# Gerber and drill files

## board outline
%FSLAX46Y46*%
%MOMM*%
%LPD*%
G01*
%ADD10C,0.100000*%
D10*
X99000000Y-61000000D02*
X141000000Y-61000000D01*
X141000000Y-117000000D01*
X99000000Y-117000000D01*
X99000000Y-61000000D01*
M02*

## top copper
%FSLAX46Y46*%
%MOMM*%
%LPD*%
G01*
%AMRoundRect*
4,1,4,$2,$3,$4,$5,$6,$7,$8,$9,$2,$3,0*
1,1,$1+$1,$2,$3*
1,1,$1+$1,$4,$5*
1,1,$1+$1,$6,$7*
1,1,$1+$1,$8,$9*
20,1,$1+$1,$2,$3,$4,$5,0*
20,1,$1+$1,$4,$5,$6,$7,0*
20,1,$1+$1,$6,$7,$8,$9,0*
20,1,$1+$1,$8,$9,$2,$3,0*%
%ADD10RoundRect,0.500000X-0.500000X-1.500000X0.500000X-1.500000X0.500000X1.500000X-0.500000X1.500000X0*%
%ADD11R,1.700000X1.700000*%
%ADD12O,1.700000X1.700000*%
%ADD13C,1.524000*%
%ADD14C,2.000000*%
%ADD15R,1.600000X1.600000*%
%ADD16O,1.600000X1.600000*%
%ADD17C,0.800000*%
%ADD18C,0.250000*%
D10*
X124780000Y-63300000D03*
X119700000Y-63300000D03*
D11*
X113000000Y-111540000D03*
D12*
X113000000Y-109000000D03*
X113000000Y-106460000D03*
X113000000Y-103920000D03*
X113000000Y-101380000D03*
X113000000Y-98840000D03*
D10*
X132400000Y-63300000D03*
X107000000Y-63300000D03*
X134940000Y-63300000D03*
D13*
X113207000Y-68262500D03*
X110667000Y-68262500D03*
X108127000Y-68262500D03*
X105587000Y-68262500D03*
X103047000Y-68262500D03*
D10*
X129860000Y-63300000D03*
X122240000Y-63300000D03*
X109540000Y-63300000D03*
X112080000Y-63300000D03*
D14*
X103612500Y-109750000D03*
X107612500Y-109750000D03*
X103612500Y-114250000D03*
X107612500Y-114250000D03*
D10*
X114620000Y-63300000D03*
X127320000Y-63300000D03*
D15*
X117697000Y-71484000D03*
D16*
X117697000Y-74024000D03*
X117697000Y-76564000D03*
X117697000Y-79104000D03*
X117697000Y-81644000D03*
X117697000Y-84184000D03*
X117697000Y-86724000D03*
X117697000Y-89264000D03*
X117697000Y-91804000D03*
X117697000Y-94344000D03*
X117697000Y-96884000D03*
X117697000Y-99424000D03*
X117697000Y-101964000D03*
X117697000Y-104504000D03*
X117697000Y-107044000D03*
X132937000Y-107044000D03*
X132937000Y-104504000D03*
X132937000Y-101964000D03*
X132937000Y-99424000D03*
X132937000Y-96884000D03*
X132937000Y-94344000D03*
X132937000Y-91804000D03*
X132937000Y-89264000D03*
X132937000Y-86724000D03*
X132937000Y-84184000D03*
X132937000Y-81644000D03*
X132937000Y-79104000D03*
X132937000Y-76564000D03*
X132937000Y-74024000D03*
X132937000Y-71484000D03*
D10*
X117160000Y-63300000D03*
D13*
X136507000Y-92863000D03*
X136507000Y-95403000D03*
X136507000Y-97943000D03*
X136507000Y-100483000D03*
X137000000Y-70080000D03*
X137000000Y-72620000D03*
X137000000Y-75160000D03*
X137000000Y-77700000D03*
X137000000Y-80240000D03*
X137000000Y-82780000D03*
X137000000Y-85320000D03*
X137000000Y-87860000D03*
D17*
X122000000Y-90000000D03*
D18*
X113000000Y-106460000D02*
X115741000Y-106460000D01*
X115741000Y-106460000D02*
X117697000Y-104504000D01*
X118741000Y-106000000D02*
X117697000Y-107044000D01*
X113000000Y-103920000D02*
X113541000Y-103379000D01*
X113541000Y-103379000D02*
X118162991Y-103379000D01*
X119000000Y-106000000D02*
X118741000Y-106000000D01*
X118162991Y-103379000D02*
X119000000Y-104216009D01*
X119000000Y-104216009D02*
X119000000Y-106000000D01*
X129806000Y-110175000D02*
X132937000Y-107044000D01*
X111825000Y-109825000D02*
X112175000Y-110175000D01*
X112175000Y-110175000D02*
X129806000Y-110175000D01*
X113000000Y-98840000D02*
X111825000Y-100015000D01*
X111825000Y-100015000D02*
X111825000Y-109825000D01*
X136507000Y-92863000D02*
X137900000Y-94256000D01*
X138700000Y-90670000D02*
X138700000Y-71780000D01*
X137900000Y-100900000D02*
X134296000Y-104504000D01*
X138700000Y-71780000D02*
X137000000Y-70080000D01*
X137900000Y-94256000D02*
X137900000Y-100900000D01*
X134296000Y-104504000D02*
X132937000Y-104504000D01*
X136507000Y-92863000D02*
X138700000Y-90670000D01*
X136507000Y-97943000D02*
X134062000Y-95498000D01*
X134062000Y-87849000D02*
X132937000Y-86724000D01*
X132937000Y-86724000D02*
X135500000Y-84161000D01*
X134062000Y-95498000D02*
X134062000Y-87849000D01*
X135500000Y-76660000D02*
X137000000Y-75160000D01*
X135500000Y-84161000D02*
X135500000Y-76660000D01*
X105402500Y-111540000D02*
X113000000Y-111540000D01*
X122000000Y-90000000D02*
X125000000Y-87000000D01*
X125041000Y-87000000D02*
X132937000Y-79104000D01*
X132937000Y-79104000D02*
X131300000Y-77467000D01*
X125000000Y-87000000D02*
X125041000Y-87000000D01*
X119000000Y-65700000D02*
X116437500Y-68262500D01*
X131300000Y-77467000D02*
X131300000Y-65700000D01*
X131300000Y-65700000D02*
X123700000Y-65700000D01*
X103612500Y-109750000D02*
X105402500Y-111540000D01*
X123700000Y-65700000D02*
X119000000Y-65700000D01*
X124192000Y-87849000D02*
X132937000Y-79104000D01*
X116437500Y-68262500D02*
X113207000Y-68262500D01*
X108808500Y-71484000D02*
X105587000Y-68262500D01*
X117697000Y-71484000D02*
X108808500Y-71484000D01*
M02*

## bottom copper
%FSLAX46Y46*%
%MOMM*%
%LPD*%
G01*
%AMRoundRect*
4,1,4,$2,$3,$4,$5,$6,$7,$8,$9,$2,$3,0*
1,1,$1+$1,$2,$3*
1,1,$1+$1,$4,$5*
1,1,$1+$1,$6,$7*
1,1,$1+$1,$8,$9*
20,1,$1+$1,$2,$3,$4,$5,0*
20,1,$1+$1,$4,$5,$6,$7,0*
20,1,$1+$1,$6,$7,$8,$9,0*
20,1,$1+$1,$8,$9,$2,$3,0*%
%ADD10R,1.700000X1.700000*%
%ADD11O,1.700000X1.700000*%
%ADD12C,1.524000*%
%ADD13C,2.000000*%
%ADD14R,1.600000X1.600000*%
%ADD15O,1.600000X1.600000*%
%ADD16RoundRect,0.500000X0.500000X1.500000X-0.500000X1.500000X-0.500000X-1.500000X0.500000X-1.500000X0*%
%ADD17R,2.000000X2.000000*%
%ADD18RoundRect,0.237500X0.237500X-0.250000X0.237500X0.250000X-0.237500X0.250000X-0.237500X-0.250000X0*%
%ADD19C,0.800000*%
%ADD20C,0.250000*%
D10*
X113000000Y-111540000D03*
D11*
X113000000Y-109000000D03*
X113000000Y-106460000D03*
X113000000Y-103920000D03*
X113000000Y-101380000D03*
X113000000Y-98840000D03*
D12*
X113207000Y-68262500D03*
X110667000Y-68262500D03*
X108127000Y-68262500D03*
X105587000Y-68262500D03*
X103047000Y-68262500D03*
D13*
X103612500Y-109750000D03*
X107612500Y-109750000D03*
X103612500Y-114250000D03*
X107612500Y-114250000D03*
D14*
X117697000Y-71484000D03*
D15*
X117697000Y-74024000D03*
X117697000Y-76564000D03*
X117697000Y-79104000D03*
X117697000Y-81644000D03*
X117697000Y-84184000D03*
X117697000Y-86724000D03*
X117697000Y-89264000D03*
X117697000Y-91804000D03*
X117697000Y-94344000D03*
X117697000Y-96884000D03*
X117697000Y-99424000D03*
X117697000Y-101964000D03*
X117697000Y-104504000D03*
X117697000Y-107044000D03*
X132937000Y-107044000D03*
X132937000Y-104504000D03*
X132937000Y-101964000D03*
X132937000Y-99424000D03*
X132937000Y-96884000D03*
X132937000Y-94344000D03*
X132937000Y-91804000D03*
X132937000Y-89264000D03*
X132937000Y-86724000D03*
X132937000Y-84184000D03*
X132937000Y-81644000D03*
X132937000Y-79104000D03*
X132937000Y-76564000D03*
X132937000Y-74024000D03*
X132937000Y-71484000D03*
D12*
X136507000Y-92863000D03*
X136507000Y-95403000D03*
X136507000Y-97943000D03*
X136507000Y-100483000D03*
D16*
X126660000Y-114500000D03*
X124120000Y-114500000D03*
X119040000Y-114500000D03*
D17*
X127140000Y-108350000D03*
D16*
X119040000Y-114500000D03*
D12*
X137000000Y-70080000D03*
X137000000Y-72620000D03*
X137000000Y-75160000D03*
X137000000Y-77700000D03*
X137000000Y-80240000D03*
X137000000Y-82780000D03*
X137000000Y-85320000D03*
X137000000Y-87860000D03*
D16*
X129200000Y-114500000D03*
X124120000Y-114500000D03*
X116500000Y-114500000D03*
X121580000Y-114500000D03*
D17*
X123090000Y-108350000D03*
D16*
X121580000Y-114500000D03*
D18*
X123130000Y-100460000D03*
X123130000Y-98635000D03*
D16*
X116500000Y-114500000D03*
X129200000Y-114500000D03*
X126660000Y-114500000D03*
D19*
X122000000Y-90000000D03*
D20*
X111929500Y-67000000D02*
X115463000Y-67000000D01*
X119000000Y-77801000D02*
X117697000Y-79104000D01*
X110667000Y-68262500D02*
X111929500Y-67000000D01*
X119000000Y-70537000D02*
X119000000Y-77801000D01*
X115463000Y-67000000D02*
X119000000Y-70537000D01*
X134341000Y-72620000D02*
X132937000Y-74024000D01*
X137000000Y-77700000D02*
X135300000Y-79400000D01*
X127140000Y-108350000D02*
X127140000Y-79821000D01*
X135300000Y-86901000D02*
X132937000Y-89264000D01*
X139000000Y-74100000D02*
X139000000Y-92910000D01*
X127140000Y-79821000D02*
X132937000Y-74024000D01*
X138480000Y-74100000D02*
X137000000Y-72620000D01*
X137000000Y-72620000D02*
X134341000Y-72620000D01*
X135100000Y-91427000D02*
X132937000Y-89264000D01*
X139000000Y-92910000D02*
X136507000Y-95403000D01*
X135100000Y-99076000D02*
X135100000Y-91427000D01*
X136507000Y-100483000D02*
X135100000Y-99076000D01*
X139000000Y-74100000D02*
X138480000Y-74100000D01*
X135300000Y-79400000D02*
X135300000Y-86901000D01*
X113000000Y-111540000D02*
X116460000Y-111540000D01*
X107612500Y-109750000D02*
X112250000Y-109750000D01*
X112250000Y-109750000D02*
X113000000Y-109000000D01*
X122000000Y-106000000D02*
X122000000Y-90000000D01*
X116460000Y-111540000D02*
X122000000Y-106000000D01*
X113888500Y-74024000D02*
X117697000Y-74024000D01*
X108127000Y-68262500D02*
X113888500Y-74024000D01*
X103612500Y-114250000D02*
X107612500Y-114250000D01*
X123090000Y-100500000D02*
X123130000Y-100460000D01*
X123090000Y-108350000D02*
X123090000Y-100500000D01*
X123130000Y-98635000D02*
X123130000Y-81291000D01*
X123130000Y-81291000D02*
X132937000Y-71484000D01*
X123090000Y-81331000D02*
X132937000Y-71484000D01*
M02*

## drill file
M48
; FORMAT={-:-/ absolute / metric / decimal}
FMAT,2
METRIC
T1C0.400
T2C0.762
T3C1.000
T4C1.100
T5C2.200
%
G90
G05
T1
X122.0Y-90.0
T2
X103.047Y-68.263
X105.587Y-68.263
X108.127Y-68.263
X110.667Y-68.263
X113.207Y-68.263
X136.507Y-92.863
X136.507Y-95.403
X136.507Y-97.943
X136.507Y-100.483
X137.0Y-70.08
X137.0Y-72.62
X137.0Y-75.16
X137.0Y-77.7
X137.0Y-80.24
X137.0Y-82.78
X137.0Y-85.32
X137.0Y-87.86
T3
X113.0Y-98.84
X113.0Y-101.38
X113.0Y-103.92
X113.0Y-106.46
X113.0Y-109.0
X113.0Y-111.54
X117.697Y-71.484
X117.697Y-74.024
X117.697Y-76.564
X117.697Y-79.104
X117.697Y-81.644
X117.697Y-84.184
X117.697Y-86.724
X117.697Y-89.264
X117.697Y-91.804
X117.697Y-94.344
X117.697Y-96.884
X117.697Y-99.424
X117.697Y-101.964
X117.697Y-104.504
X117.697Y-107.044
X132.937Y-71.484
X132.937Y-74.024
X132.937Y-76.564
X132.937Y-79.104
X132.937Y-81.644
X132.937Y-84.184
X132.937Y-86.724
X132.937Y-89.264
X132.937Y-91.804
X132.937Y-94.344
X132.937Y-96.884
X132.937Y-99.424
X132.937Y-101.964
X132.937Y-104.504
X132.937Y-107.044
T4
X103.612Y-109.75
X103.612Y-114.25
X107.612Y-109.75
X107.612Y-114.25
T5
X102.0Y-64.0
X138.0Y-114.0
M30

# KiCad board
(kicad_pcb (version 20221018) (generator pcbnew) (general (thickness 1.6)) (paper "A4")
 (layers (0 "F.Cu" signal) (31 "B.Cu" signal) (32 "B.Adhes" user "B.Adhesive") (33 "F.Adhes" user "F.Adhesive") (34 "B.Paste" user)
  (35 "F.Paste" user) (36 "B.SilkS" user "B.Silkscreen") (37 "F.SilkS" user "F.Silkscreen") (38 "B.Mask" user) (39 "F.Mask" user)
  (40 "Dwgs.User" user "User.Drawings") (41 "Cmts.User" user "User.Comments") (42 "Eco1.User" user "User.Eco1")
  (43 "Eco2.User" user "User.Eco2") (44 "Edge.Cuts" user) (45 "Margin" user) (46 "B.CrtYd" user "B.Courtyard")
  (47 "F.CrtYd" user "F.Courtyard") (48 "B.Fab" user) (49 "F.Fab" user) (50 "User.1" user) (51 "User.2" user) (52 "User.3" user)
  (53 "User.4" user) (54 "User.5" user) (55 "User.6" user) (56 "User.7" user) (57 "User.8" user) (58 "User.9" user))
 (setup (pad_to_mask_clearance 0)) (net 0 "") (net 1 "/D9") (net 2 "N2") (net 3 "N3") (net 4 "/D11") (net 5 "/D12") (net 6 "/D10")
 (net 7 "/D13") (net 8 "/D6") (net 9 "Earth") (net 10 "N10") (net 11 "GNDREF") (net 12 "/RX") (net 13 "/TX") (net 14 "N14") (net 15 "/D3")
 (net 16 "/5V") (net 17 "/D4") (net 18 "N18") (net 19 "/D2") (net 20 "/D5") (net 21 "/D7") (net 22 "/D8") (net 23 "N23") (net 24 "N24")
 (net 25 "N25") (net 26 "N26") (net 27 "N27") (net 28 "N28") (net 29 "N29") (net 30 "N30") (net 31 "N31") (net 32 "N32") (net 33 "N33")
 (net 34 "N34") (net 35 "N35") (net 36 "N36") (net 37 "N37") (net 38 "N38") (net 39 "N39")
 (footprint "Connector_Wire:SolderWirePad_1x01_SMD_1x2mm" (layer "F.Cu") (at 124.78 63.3)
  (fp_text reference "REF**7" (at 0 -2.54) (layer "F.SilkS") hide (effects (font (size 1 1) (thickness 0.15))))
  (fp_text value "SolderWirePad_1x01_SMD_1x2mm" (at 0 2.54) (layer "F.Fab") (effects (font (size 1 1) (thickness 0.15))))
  (pad "1" smd roundrect (at 0 0) (size 2 4) (layers "F.Cu" "F.Paste" "F.Mask") (roundrect_rratio 0.25) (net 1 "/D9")))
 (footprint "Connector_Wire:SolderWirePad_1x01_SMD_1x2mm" (layer "F.Cu") (at 119.7 63.3)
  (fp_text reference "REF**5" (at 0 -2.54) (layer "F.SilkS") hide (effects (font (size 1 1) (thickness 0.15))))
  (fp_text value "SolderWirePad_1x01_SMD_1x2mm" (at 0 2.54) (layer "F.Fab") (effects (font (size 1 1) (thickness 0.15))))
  (pad "1" smd roundrect (at 0 0) (size 2 4) (layers "F.Cu" "F.Paste" "F.Mask") (roundrect_rratio 0.25)))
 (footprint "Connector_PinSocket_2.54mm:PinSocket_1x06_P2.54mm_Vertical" (layer "F.Cu") (at 113 111.54 180)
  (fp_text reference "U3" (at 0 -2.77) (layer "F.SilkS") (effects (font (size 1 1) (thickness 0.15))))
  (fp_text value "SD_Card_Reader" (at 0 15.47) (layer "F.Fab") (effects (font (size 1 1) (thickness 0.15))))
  (pad "1" thru_hole rect (at 0 0 180) (size 1.7 1.7) (drill 1) (layers "*.Cu" "*.Mask") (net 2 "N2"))
  (pad "2" thru_hole oval (at 0 2.54 180) (size 1.7 1.7) (drill 1) (layers "*.Cu" "*.Mask") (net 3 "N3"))
  (pad "3" thru_hole oval (at 0 5.08 180) (size 1.7 1.7) (drill 1) (layers "*.Cu" "*.Mask") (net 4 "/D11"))
  (pad "4" thru_hole oval (at 0 7.62 180) (size 1.7 1.7) (drill 1) (layers "*.Cu" "*.Mask") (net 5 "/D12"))
  (pad "5" thru_hole oval (at 0 10.16 180) (size 1.7 1.7) (drill 1) (layers "*.Cu" "*.Mask") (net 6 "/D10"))
  (pad "6" thru_hole oval (at 0 12.7 180) (size 1.7 1.7) (drill 1) (layers "*.Cu" "*.Mask") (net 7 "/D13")))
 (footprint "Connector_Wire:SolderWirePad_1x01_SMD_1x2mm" (layer "F.Cu") (at 132.4 63.3)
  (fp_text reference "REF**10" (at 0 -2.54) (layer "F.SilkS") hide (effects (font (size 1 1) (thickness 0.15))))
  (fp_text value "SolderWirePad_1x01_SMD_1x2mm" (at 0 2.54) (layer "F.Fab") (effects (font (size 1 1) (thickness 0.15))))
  (pad "1" smd roundrect (at 0 0) (size 2 4) (layers "F.Cu" "F.Paste" "F.Mask") (roundrect_rratio 0.25) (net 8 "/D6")))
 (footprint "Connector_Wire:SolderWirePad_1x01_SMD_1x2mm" (layer "F.Cu") (at 107 63.3)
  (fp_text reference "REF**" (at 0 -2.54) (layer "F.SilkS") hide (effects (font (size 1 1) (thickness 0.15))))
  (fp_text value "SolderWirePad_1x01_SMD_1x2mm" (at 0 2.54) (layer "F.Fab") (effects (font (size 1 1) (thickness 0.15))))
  (pad "1" smd roundrect (at 0 0) (size 2 4) (layers "F.Cu" "F.Paste" "F.Mask") (roundrect_rratio 0.25) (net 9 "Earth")))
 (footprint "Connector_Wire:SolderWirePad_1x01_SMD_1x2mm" (layer "F.Cu") (at 134.94 63.3)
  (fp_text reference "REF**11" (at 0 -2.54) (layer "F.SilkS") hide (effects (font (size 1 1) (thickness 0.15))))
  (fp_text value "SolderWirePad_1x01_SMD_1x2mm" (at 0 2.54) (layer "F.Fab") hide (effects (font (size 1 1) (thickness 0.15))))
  (pad "1" smd roundrect (at 0 0) (size 2 4) (layers "F.Cu" "F.Paste" "F.Mask") (roundrect_rratio 0.25)))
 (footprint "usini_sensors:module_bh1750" (layer "F.Cu") (at 103.047 68.2625 -90)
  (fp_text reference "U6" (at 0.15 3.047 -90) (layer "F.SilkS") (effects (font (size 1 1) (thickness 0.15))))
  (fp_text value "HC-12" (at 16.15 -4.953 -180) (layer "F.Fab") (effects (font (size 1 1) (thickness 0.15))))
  (pad "1" thru_hole circle (at 0 -10.16 270) (size 1.524 1.524) (drill 0.762) (layers "*.Cu" "*.Mask") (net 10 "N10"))
  (pad "2" thru_hole circle (at 0 -7.62 270) (size 1.524 1.524) (drill 0.762) (layers "*.Cu" "*.Mask") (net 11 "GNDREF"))
  (pad "3" thru_hole circle (at 0 -5.08 270) (size 1.524 1.524) (drill 0.762) (layers "*.Cu" "*.Mask") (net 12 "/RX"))
  (pad "4" thru_hole circle (at 0 -2.54 270) (size 1.524 1.524) (drill 0.762) (layers "*.Cu" "*.Mask") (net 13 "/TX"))
  (pad "5" thru_hole circle (at 0 0 270) (size 1.524 1.524) (drill 0.762) (layers "*.Cu" "*.Mask") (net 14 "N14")))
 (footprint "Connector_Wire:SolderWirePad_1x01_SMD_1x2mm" (layer "F.Cu") (at 129.86 63.3)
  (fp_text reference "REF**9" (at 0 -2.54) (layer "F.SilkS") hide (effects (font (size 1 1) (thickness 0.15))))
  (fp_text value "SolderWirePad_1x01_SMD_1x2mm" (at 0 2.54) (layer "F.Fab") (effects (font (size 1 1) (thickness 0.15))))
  (pad "1" smd roundrect (at 0 0) (size 2 4) (layers "F.Cu" "F.Paste" "F.Mask") (roundrect_rratio 0.25) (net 9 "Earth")))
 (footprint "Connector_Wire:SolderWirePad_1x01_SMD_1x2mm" (layer "F.Cu") (at 122.24 63.3)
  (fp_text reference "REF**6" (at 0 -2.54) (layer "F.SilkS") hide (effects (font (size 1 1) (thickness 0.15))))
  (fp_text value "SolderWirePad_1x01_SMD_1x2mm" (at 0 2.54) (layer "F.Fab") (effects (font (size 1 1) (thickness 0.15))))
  (pad "1" smd roundrect (at 0 0) (size 2 4) (layers "F.Cu" "F.Paste" "F.Mask") (roundrect_rratio 0.25) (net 9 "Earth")))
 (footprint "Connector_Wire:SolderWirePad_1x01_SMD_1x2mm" (layer "F.Cu") (at 109.54 63.3)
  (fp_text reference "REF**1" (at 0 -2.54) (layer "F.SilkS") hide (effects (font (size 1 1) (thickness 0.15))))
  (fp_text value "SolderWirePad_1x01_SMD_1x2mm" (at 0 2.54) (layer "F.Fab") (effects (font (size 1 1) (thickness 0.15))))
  (pad "1" smd roundrect (at 0 0) (size 2 4) (layers "F.Cu" "F.Paste" "F.Mask") (roundrect_rratio 0.25) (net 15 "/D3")))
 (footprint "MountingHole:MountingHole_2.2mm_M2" (layer "F.Cu") (at 138 114)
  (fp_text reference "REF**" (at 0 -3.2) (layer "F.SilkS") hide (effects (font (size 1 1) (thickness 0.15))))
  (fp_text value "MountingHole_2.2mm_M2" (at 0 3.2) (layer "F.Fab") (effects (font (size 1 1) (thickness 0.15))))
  (pad "" np_thru_hole circle (at 0 0) (size 2.2 2.2) (drill 2.2) (layers "*.Cu" "*.Mask")))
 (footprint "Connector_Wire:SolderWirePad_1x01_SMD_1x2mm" (layer "F.Cu") (at 112.08 63.3)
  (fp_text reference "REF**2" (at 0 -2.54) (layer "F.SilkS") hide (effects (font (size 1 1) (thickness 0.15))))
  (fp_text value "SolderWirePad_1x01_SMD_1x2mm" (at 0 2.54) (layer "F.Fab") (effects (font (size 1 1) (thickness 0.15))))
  (pad "1" smd roundrect (at 0 0) (size 2 4) (layers "F.Cu" "F.Paste" "F.Mask") (roundrect_rratio 0.25)))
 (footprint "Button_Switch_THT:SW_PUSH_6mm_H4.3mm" (layer "F.Cu") (at 101.1125 109.75)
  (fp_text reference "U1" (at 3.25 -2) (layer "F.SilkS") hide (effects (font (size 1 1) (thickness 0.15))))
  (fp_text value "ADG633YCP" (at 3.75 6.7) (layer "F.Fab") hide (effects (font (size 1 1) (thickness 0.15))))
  (pad "1" thru_hole circle (at 2.5 0 90) (size 2 2) (drill 1.1) (layers "*.Cu" "*.Mask") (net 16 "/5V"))
  (pad "1" thru_hole circle (at 6.5 0 90) (size 2 2) (drill 1.1) (layers "*.Cu" "*.Mask") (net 16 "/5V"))
  (pad "2" thru_hole circle (at 2.5 4.5 90) (size 2 2) (drill 1.1) (layers "*.Cu" "*.Mask") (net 8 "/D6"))
  (pad "2" thru_hole circle (at 6.5 4.5 90) (size 2 2) (drill 1.1) (layers "*.Cu" "*.Mask") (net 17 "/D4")))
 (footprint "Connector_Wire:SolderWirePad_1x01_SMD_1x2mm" (layer "F.Cu") (at 114.62 63.3)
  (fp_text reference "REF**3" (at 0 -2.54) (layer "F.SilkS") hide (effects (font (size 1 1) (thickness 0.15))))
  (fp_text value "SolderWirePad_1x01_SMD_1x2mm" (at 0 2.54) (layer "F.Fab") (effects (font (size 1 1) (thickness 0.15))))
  (pad "1" smd roundrect (at 0 0) (size 2 4) (layers "F.Cu" "F.Paste" "F.Mask") (roundrect_rratio 0.25) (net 9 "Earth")))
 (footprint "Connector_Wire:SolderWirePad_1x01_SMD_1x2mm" (layer "F.Cu") (at 127.32 63.3)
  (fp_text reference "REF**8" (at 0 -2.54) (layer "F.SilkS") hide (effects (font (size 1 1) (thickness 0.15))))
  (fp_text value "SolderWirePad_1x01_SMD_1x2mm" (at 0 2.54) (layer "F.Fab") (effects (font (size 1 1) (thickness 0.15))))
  (pad "1" smd roundrect (at 0 0) (size 2 4) (layers "F.Cu" "F.Paste" "F.Mask") (roundrect_rratio 0.25)))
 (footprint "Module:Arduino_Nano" (layer "F.Cu") (at 117.697 71.484)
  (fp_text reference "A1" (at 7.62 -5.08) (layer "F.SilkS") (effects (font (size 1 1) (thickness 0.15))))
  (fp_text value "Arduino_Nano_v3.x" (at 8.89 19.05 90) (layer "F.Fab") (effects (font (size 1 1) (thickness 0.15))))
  (pad "1" thru_hole rect (at 0 0) (size 1.6 1.6) (drill 1) (layers "*.Cu" "*.Mask") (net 13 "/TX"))
  (pad "2" thru_hole oval (at 0 2.54) (size 1.6 1.6) (drill 1) (layers "*.Cu" "*.Mask") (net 12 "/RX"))
  (pad "3" thru_hole oval (at 0 5.08) (size 1.6 1.6) (drill 1) (layers "*.Cu" "*.Mask") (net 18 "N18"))
  (pad "4" thru_hole oval (at 0 7.62) (size 1.6 1.6) (drill 1) (layers "*.Cu" "*.Mask") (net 9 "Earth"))
  (pad "5" thru_hole oval (at 0 10.16) (size 1.6 1.6) (drill 1) (layers "*.Cu" "*.Mask") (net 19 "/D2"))
  (pad "6" thru_hole oval (at 0 12.7) (size 1.6 1.6) (drill 1) (layers "*.Cu" "*.Mask") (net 15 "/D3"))
  (pad "7" thru_hole oval (at 0 15.24) (size 1.6 1.6) (drill 1) (layers "*.Cu" "*.Mask") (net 17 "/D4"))
  (pad "8" thru_hole oval (at 0 17.78) (size 1.6 1.6) (drill 1) (layers "*.Cu" "*.Mask") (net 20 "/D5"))
  (pad "9" thru_hole oval (at 0 20.32) (size 1.6 1.6) (drill 1) (layers "*.Cu" "*.Mask") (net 8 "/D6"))
  (pad "10" thru_hole oval (at 0 22.86) (size 1.6 1.6) (drill 1) (layers "*.Cu" "*.Mask") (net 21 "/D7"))
  (pad "11" thru_hole oval (at 0 25.4) (size 1.6 1.6) (drill 1) (layers "*.Cu" "*.Mask") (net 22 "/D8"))
  (pad "12" thru_hole oval (at 0 27.94) (size 1.6 1.6) (drill 1) (layers "*.Cu" "*.Mask") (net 1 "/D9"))
  (pad "13" thru_hole oval (at 0 30.48) (size 1.6 1.6) (drill 1) (layers "*.Cu" "*.Mask") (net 6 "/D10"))
  (pad "14" thru_hole oval (at 0 33.02) (size 1.6 1.6) (drill 1) (layers "*.Cu" "*.Mask") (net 4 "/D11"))
  (pad "15" thru_hole oval (at 0 35.56) (size 1.6 1.6) (drill 1) (layers "*.Cu" "*.Mask") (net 5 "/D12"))
  (pad "16" thru_hole oval (at 15.24 35.56) (size 1.6 1.6) (drill 1) (layers "*.Cu" "*.Mask") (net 7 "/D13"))
  (pad "17" thru_hole oval (at 15.24 33.02) (size 1.6 1.6) (drill 1) (layers "*.Cu" "*.Mask") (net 10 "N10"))
  (pad "18" thru_hole oval (at 15.24 30.48) (size 1.6 1.6) (drill 1) (layers "*.Cu" "*.Mask") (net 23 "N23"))
  (pad "19" thru_hole oval (at 15.24 27.94) (size 1.6 1.6) (drill 1) (layers "*.Cu" "*.Mask") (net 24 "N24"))
  (pad "20" thru_hole oval (at 15.24 25.4) (size 1.6 1.6) (drill 1) (layers "*.Cu" "*.Mask") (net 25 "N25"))
  (pad "21" thru_hole oval (at 15.24 22.86) (size 1.6 1.6) (drill 1) (layers "*.Cu" "*.Mask") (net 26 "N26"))
  (pad "22" thru_hole oval (at 15.24 20.32) (size 1.6 1.6) (drill 1) (layers "*.Cu" "*.Mask") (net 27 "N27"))
  (pad "23" thru_hole oval (at 15.24 17.78) (size 1.6 1.6) (drill 1) (layers "*.Cu" "*.Mask") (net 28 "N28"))
  (pad "24" thru_hole oval (at 15.24 15.24) (size 1.6 1.6) (drill 1) (layers "*.Cu" "*.Mask") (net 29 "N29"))
  (pad "25" thru_hole oval (at 15.24 12.7) (size 1.6 1.6) (drill 1) (layers "*.Cu" "*.Mask") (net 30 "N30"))
  (pad "26" thru_hole oval (at 15.24 10.16) (size 1.6 1.6) (drill 1) (layers "*.Cu" "*.Mask") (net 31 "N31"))
  (pad "27" thru_hole oval (at 15.24 7.62) (size 1.6 1.6) (drill 1) (layers "*.Cu" "*.Mask") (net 16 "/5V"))
  (pad "28" thru_hole oval (at 15.24 5.08) (size 1.6 1.6) (drill 1) (layers "*.Cu" "*.Mask") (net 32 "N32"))
  (pad "29" thru_hole oval (at 15.24 2.54) (size 1.6 1.6) (drill 1) (layers "*.Cu" "*.Mask") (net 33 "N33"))
  (pad "30" thru_hole oval (at 15.24 0) (size 1.6 1.6) (drill 1) (layers "*.Cu" "*.Mask") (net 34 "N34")))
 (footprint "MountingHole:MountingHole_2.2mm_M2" (layer "F.Cu") (at 102 64)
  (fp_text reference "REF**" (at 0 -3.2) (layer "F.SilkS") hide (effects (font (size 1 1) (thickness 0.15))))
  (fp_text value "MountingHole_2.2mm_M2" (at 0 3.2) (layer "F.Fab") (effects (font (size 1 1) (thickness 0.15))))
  (pad "" np_thru_hole circle (at 0 0) (size 2.2 2.2) (drill 2.2) (layers "*.Cu" "*.Mask")))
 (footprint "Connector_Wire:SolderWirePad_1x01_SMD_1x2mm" (layer "F.Cu") (at 117.16 63.3)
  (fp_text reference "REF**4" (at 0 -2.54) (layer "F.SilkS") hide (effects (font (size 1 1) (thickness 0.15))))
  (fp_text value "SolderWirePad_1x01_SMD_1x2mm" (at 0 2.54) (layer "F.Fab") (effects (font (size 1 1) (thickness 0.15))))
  (pad "1" smd roundrect (at 0 0) (size 2 4) (layers "F.Cu" "F.Paste" "F.Mask") (roundrect_rratio 0.25) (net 20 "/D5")))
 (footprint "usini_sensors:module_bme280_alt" (layer "B.Cu") (at 136.507 100.483 180)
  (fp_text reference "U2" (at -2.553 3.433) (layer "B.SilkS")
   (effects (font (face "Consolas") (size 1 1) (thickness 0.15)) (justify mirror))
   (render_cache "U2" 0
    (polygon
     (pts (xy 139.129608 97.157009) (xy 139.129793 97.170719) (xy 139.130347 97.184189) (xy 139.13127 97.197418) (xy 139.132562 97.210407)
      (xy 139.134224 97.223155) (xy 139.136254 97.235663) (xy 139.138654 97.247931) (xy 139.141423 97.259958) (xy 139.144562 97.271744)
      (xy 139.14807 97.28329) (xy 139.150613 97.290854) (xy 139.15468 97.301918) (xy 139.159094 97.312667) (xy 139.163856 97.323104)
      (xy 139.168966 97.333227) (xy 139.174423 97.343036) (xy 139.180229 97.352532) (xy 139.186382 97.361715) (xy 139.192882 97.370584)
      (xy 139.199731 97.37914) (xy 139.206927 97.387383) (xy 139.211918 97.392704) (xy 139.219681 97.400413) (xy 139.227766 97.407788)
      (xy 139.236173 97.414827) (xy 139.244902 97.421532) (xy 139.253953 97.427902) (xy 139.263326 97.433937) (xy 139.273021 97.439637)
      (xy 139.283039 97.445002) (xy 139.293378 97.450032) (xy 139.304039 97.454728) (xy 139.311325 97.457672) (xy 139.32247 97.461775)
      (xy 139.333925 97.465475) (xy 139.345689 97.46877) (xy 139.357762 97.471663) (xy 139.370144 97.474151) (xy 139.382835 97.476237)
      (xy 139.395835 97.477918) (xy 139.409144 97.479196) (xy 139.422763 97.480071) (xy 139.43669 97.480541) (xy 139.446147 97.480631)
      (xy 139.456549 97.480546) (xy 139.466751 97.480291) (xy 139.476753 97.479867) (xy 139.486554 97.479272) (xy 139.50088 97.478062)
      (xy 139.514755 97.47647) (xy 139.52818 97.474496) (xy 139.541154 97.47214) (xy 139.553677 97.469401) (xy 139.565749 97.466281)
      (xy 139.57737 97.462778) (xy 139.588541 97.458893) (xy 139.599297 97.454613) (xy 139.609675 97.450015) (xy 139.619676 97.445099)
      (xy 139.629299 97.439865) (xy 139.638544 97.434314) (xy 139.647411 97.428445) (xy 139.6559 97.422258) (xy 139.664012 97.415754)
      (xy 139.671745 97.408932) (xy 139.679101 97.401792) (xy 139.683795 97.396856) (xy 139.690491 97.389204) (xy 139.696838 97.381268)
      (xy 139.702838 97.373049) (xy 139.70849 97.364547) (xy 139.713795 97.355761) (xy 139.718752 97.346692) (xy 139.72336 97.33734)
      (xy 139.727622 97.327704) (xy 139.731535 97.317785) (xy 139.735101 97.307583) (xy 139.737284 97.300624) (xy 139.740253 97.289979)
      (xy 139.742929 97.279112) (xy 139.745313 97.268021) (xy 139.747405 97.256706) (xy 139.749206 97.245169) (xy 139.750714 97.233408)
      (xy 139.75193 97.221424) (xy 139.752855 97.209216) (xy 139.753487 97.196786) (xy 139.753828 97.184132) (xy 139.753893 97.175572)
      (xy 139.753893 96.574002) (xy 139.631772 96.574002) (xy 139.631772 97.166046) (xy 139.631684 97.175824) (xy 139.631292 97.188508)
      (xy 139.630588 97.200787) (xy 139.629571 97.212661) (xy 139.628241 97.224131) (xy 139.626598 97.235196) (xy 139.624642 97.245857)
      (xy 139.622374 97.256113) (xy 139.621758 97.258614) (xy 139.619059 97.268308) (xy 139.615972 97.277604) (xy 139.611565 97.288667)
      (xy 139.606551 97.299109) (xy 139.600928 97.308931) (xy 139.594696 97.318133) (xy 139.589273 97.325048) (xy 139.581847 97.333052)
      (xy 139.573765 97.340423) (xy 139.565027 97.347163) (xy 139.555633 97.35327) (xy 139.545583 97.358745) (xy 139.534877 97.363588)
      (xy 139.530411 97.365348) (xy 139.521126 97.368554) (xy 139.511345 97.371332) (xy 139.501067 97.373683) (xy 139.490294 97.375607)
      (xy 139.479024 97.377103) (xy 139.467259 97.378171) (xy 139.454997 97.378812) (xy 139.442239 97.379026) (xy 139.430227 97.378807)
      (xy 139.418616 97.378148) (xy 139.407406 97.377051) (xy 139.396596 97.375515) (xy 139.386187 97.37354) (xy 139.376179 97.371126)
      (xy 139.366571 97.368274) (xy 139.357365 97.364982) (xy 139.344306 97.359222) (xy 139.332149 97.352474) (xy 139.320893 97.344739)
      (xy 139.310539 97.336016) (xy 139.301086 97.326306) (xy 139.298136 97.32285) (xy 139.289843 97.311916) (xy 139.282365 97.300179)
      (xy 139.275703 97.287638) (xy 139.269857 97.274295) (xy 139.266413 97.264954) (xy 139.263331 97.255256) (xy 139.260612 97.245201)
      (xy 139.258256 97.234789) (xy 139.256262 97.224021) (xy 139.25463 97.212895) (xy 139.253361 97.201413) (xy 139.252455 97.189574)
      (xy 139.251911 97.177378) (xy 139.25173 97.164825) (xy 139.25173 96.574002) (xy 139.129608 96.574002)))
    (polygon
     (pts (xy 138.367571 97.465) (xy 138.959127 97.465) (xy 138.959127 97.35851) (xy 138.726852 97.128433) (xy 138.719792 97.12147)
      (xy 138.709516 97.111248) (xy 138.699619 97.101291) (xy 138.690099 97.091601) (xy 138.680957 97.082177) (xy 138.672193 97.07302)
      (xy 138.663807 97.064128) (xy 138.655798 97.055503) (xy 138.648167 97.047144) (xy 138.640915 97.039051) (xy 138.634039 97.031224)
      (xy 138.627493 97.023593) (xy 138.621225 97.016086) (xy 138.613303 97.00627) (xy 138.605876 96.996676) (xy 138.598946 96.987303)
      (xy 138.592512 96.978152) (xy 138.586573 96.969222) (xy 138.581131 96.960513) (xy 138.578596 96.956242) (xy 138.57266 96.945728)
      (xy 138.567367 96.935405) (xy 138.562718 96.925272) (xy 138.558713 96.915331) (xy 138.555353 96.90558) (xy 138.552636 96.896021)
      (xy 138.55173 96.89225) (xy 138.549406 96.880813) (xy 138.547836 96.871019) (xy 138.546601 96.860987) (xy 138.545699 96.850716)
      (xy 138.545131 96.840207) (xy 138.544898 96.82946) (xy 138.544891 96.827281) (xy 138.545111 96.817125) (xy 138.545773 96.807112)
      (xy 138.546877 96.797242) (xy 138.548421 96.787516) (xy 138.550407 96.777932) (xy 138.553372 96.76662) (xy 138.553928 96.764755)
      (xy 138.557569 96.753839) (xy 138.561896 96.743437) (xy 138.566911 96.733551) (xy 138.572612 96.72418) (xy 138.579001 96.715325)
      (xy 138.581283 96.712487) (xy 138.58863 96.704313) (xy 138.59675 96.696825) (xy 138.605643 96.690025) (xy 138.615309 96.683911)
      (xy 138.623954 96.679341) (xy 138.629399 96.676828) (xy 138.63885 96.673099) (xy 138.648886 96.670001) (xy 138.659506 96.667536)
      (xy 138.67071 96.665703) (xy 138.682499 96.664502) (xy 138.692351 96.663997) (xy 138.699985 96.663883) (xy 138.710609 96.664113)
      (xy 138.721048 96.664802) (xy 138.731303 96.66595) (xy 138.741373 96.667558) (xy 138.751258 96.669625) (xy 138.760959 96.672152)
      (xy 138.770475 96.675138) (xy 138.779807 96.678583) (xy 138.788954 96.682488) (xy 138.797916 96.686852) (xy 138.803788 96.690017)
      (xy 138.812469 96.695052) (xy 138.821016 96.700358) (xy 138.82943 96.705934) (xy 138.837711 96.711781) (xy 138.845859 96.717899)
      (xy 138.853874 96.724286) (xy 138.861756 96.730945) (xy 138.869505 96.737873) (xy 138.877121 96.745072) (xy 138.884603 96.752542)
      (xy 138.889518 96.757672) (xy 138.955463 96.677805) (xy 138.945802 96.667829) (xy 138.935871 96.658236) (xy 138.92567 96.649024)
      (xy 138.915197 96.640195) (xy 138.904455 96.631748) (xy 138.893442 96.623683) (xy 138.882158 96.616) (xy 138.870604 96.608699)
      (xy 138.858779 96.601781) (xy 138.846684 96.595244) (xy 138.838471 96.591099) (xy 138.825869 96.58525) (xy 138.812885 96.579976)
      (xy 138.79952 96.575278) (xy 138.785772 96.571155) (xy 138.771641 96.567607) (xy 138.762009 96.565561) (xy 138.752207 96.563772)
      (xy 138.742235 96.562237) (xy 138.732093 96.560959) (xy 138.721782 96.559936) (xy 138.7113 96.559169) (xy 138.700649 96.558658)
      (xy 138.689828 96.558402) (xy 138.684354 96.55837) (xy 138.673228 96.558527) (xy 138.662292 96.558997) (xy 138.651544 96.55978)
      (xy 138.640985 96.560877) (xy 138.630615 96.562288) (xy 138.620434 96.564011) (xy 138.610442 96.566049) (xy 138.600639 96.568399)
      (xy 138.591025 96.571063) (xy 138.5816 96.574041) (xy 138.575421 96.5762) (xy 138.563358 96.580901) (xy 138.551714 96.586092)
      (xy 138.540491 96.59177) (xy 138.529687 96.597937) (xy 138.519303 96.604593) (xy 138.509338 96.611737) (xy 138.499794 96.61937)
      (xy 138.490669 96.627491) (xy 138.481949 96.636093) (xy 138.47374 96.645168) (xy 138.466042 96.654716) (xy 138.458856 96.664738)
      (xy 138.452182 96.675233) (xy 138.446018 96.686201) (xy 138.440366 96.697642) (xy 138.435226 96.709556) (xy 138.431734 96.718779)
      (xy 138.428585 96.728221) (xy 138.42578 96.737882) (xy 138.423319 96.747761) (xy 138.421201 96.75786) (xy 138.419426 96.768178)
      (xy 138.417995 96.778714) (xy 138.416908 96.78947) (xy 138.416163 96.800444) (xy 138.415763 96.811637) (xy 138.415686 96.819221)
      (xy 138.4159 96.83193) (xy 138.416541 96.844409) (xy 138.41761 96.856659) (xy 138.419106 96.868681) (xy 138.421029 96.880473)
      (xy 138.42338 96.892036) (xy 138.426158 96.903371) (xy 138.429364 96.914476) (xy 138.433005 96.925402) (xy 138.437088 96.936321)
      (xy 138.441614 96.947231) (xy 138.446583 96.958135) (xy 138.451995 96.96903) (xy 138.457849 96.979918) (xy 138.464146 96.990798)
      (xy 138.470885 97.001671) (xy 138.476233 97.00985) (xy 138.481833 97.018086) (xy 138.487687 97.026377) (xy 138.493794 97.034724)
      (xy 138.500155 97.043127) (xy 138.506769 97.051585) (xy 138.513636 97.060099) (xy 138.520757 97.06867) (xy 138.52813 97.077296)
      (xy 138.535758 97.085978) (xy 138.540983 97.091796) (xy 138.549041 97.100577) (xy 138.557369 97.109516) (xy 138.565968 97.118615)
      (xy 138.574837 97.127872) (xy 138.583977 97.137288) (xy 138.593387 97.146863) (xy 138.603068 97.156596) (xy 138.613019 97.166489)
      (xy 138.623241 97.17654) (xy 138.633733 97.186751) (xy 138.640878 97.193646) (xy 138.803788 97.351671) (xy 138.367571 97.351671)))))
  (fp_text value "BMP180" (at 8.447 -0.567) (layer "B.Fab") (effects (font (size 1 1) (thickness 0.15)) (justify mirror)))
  (pad "1" thru_hole circle (at 0 7.62 180) (size 1.524 1.524) (drill 0.762) (layers "*.Cu" "*.Mask") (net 29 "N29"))
  (pad "2" thru_hole circle (at 0 5.08 180) (size 1.524 1.524) (drill 0.762) (layers "*.Cu" "*.Mask") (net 28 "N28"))
  (pad "3" thru_hole circle (at 0 2.54 180) (size 1.524 1.524) (drill 0.762) (layers "*.Cu" "*.Mask") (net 11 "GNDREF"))
  (pad "4" thru_hole circle (at 0 0 180) (size 1.524 1.524) (drill 0.762) (layers "*.Cu" "*.Mask") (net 10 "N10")))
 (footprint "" (layer "B.Cu") (at 126.66 114.5 180)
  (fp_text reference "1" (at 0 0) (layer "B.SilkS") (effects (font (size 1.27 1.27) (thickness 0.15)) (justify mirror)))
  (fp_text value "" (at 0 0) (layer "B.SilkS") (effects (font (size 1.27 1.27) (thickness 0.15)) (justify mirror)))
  (pad "1" smd roundrect (at 0 0 180) (size 2 4) (layers "B.Cu" "B.Paste" "B.Mask") (roundrect_rratio 0.25)))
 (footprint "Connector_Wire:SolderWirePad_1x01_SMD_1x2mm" (layer "B.Cu") (at 124.12 114.5 180)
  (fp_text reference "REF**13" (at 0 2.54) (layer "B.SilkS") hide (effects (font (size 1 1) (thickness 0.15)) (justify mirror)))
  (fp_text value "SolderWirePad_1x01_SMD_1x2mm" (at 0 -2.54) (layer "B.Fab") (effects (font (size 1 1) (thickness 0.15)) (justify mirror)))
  (pad "1" smd roundrect (at 0 0 180) (size 2 4) (layers "B.Cu" "B.Paste" "B.Mask") (roundrect_rratio 0.25)))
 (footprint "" (layer "B.Cu") (at 119.04 114.5 180)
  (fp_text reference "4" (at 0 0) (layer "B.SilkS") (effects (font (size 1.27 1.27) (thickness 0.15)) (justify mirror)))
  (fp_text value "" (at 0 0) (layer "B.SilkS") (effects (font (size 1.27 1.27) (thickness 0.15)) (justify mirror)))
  (pad "1" smd roundrect (at 0 0 180) (size 2 4) (layers "B.Cu" "B.Paste" "B.Mask") (roundrect_rratio 0.25)))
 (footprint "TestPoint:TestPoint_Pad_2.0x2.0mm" (layer "B.Cu") (at 127.14 108.35 -90)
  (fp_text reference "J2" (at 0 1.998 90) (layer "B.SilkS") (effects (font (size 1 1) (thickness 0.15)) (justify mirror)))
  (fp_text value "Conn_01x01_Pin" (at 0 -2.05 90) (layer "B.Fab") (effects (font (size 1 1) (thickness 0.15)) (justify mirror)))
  (pad "1" smd rect (at 0 0 270) (size 2 2) (layers "B.Cu" "B.Mask") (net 33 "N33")))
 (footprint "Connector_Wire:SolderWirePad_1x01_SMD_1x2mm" (layer "B.Cu") (at 119.04 114.5 180)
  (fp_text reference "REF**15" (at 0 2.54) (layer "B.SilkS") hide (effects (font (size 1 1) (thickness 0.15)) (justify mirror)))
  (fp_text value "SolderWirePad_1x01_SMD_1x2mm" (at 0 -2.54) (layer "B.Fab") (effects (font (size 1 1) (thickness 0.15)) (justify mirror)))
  (pad "1" smd roundrect (at 0 0 180) (size 2 4) (layers "B.Cu" "B.Paste" "B.Mask") (roundrect_rratio 0.25) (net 6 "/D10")))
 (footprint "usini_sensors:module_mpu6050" (layer "B.Cu") (at 137 87.86 180)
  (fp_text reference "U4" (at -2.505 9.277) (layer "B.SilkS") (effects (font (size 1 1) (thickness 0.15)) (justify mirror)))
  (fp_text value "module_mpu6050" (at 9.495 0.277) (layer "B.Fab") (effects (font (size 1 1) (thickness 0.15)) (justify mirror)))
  (pad "1" thru_hole circle (at 0 17.78 180) (size 1.524 1.524) (drill 0.762) (layers "*.Cu" "*.Mask") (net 10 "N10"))
  (pad "2" thru_hole circle (at 0 15.24 180) (size 1.524 1.524) (drill 0.762) (layers "*.Cu" "*.Mask") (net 11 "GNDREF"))
  (pad "3" thru_hole circle (at 0 12.7 180) (size 1.524 1.524) (drill 0.762) (layers "*.Cu" "*.Mask") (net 28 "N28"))
  (pad "4" thru_hole circle (at 0 10.16 180) (size 1.524 1.524) (drill 0.762) (layers "*.Cu" "*.Mask") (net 29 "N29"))
  (pad "5" thru_hole circle (at 0 7.62 180) (size 1.524 1.524) (drill 0.762) (layers "*.Cu" "*.Mask") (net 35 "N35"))
  (pad "6" thru_hole circle (at 0 5.08 180) (size 1.524 1.524) (drill 0.762) (layers "*.Cu" "*.Mask") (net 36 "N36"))
  (pad "7" thru_hole circle (at 0 2.54 180) (size 1.524 1.524) (drill 0.762) (layers "*.Cu" "*.Mask") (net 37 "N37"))
  (pad "8" thru_hole circle (at 0 0 180) (size 1.524 1.524) (drill 0.762) (layers "*.Cu" "*.Mask") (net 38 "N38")))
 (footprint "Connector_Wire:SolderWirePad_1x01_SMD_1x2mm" (layer "B.Cu") (at 129.2 114.5 180)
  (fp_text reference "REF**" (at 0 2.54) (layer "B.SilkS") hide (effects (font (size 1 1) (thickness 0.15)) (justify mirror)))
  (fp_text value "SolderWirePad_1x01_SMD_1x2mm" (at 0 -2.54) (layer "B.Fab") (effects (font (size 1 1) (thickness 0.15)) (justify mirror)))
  (pad "1" smd roundrect (at 0 0 180) (size 2 4) (layers "B.Cu" "B.Paste" "B.Mask") (roundrect_rratio 0.25)))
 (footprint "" (layer "B.Cu") (at 124.12 114.5 180)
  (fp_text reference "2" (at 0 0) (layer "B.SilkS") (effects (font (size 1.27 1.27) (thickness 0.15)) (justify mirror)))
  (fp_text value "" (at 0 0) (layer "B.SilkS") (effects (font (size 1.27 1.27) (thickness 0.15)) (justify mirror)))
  (pad "1" smd roundrect (at 0 0 180) (size 2 4) (layers "B.Cu" "B.Paste" "B.Mask") (roundrect_rratio 0.25)))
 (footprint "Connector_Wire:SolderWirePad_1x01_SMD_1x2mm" (layer "B.Cu") (at 116.5 114.5 180)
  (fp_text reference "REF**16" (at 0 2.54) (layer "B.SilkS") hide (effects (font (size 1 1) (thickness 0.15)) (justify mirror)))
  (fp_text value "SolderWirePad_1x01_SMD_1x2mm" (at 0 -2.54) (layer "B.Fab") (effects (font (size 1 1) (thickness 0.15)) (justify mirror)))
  (pad "1" smd roundrect (at 0 0 180) (size 2 4) (layers "B.Cu" "B.Paste" "B.Mask") (roundrect_rratio 0.25)))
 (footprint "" (layer "B.Cu") (at 121.58 114.5 180)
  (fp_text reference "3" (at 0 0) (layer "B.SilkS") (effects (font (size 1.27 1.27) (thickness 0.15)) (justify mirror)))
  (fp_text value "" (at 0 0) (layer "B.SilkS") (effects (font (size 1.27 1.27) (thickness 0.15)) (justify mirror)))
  (pad "1" smd roundrect (at 0 0 180) (size 2 4) (layers "B.Cu" "B.Paste" "B.Mask") (roundrect_rratio 0.25)))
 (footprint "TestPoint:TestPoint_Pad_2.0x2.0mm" (layer "B.Cu") (at 123.09 108.35 -90)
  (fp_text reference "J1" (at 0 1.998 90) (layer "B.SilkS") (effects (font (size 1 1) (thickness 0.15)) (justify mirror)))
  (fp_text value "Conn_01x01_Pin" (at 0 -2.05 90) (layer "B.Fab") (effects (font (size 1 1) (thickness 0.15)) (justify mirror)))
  (pad "1" smd rect (at 0 0 270) (size 2 2) (layers "B.Cu" "B.Mask") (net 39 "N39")))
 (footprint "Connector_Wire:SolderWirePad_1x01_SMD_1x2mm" (layer "B.Cu") (at 121.58 114.5 180)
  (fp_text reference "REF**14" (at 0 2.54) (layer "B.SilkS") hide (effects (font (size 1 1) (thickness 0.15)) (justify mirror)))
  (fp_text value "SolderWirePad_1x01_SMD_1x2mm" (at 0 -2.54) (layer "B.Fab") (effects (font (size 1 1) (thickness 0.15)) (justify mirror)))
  (pad "1" smd roundrect (at 0 0 180) (size 2 4) (layers "B.Cu" "B.Paste" "B.Mask") (roundrect_rratio 0.25)))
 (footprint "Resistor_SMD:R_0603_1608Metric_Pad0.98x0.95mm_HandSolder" (layer "B.Cu") (at 123.13 99.5475 90)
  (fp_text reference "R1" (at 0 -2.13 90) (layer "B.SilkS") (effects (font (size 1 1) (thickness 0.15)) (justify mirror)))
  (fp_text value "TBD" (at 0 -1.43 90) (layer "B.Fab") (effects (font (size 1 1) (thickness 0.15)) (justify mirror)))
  (pad "1" smd roundrect (at -0.9125 0 90) (size 0.975 0.95) (layers "B.Cu" "B.Paste" "B.Mask") (roundrect_rratio 0.25) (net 39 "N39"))
  (pad "2" smd roundrect (at 0.9125 0 90) (size 0.975 0.95) (layers "B.Cu" "B.Paste" "B.Mask") (roundrect_rratio 0.25) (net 34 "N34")))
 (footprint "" (layer "B.Cu") (at 116.5 114.5 180)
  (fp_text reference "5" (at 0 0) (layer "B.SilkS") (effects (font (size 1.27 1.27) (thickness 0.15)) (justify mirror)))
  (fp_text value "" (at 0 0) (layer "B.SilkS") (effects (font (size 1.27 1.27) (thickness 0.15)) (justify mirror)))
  (pad "1" smd roundrect (at 0 0 180) (size 2 4) (layers "B.Cu" "B.Paste" "B.Mask") (roundrect_rratio 0.25)))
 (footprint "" (layer "B.Cu") (at 129.2 114.5 180)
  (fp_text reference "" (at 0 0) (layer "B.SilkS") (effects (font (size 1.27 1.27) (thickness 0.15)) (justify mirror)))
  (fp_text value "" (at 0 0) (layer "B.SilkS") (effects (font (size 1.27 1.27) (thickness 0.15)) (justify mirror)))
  (pad "1" smd roundrect (at 0 0 180) (size 2 4) (layers "B.Cu" "B.Paste" "B.Mask") (roundrect_rratio 0.25)))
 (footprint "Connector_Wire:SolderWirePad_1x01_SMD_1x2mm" (layer "B.Cu") (at 126.66 114.5 180)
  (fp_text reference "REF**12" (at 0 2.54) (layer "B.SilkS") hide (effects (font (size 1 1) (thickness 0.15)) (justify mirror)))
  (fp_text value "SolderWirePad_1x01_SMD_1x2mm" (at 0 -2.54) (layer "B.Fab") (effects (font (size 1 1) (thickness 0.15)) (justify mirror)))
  (pad "1" smd roundrect (at 0 0 180) (size 2 4) (layers "B.Cu" "B.Paste" "B.Mask") (roundrect_rratio 0.25)))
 (gr_rect (start 99 61) (end 141 117) (stroke (width 0.1) (type default)) (fill none) (layer "Edge.Cuts"))
 (segment (start 111.9295 67) (end 115.463 67) (width 0.25) (layer "B.Cu") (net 9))
 (segment (start 119 77.801) (end 117.697 79.104) (width 0.25) (layer "B.Cu") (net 9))
 (segment (start 110.667 68.2625) (end 111.9295 67) (width 0.25) (layer "B.Cu") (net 9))
 (segment (start 119 70.537) (end 119 77.801) (width 0.25) (layer "B.Cu") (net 9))
 (segment (start 115.463 67) (end 119 70.537) (width 0.25) (layer "B.Cu") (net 9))
 (segment (start 113 106.46) (end 115.741 106.46) (width 0.25) (layer "F.Cu") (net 4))
 (segment (start 115.741 106.46) (end 117.697 104.504) (width 0.25) (layer "F.Cu") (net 4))
 (segment (start 118.741 106) (end 117.697 107.044) (width 0.25) (layer "F.Cu") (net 5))
 (segment (start 113 103.92) (end 113.541 103.379) (width 0.25) (layer "F.Cu") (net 5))
 (segment (start 113.541 103.379) (end 118.162991 103.379) (width 0.25) (layer "F.Cu") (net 5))
 (segment (start 119 106) (end 118.741 106) (width 0.25) (layer "F.Cu") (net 5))
 (segment (start 118.162991 103.379) (end 119 104.216009) (width 0.25) (layer "F.Cu") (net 5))
 (segment (start 119 104.216009) (end 119 106) (width 0.25) (layer "F.Cu") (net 5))
 (segment (start 129.806 110.175) (end 132.937 107.044) (width 0.25) (layer "F.Cu") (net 7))
 (segment (start 111.825 109.825) (end 112.175 110.175) (width 0.25) (layer "F.Cu") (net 7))
 (segment (start 112.175 110.175) (end 129.806 110.175) (width 0.25) (layer "F.Cu") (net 7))
 (segment (start 113 98.84) (end 111.825 100.015) (width 0.25) (layer "F.Cu") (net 7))
 (segment (start 111.825 100.015) (end 111.825 109.825) (width 0.25) (layer "F.Cu") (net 7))
 (segment (start 136.507 92.863) (end 137.9 94.256) (width 0.25) (layer "F.Cu") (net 10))
 (segment (start 138.7 90.67) (end 138.7 71.78) (width 0.25) (layer "F.Cu") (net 10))
 (segment (start 137.9 100.9) (end 134.296 104.504) (width 0.25) (layer "F.Cu") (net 10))
 (segment (start 138.7 71.78) (end 137 70.08) (width 0.25) (layer "F.Cu") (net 10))
 (segment (start 137.9 94.256) (end 137.9 100.9) (width 0.25) (layer "F.Cu") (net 10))
 (segment (start 134.296 104.504) (end 132.937 104.504) (width 0.25) (layer "F.Cu") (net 10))
 (segment (start 136.507 92.863) (end 138.7 90.67) (width 0.25) (layer "F.Cu") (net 10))
 (segment (start 134.341 72.62) (end 132.937 74.024) (width 0.25) (layer "B.Cu") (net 28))
 (segment (start 137 77.7) (end 135.3 79.4) (width 0.25) (layer "B.Cu") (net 28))
 (segment (start 127.14 108.35) (end 127.14 79.821) (width 0.25) (layer "B.Cu") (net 28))
 (segment (start 135.3 86.901) (end 132.937 89.264) (width 0.25) (layer "B.Cu") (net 28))
 (segment (start 139 74.1) (end 139 92.91) (width 0.25) (layer "B.Cu") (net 28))
 (segment (start 127.14 79.821) (end 132.937 74.024) (width 0.25) (layer "B.Cu") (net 28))
 (segment (start 138.48 74.1) (end 137 72.62) (width 0.25) (layer "B.Cu") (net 28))
 (segment (start 137 72.62) (end 134.341 72.62) (width 0.25) (layer "B.Cu") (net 28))
 (segment (start 135.1 91.427) (end 132.937 89.264) (width 0.25) (layer "B.Cu") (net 28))
 (segment (start 139 92.91) (end 136.507 95.403) (width 0.25) (layer "B.Cu") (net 28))
 (segment (start 135.1 99.076) (end 135.1 91.427) (width 0.25) (layer "B.Cu") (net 28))
 (segment (start 136.507 100.483) (end 135.1 99.076) (width 0.25) (layer "B.Cu") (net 28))
 (segment (start 139 74.1) (end 138.48 74.1) (width 0.25) (layer "B.Cu") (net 28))
 (segment (start 135.3 79.4) (end 135.3 86.901) (width 0.25) (layer "B.Cu") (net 28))
 (segment (start 136.507 97.943) (end 134.062 95.498) (width 0.25) (layer "F.Cu") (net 29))
 (segment (start 134.062 87.849) (end 132.937 86.724) (width 0.25) (layer "F.Cu") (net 29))
 (segment (start 132.937 86.724) (end 135.5 84.161) (width 0.25) (layer "F.Cu") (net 29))
 (segment (start 134.062 95.498) (end 134.062 87.849) (width 0.25) (layer "F.Cu") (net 29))
 (segment (start 135.5 76.66) (end 137 75.16) (width 0.25) (layer "F.Cu") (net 29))
 (segment (start 135.5 84.161) (end 135.5 76.66) (width 0.25) (layer "F.Cu") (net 29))
 (segment (start 105.4025 111.54) (end 113 111.54) (width 0.25) (layer "F.Cu") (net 16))
 (segment (start 122 90) (end 125 87) (width 0.25) (layer "F.Cu") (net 16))
 (segment (start 125.041 87) (end 132.937 79.104) (width 0.25) (layer "F.Cu") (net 16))
 (segment (start 132.937 79.104) (end 131.3 77.467) (width 0.25) (layer "F.Cu") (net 16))
 (segment (start 125 87) (end 125.041 87) (width 0.25) (layer "F.Cu") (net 16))
 (segment (start 119 65.7) (end 116.4375 68.2625) (width 0.25) (layer "F.Cu") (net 16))
 (segment (start 131.3 77.467) (end 131.3 65.7) (width 0.25) (layer "F.Cu") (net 16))
 (segment (start 131.3 65.7) (end 123.7 65.7) (width 0.25) (layer "F.Cu") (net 16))
 (segment (start 103.6125 109.75) (end 105.4025 111.54) (width 0.25) (layer "F.Cu") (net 16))
 (segment (start 123.7 65.7) (end 119 65.7) (width 0.25) (layer "F.Cu") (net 16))
 (segment (start 124.192 87.849) (end 132.937 79.104) (width 0.25) (layer "F.Cu") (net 16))
 (segment (start 116.4375 68.2625) (end 113.207 68.2625) (width 0.25) (layer "F.Cu") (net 16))
 (via (at 122 90) (size 0.8) (drill 0.4) (layers "F.Cu" "B.Cu") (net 16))
 (segment (start 113 111.54) (end 116.46 111.54) (width 0.25) (layer "B.Cu") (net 16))
 (segment (start 107.6125 109.75) (end 112.25 109.75) (width 0.25) (layer "B.Cu") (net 16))
 (segment (start 112.25 109.75) (end 113 109) (width 0.25) (layer "B.Cu") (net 16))
 (segment (start 122 106) (end 122 90) (width 0.25) (layer "B.Cu") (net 16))
 (segment (start 116.46 111.54) (end 122 106) (width 0.25) (layer "B.Cu") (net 16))
 (segment (start 108.8085 71.484) (end 105.587 68.2625) (width 0.25) (layer "F.Cu") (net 13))
 (segment (start 117.697 71.484) (end 108.8085 71.484) (width 0.25) (layer "F.Cu") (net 13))
 (segment (start 113.8885 74.024) (end 117.697 74.024) (width 0.25) (layer "B.Cu") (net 12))
 (segment (start 108.127 68.2625) (end 113.8885 74.024) (width 0.25) (layer "B.Cu") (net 12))
 (segment (start 103.6125 114.25) (end 107.6125 114.25) (width 0.25) (layer "B.Cu") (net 8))
 (segment (start 123.09 100.5) (end 123.13 100.46) (width 0.25) (layer "B.Cu") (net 39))
 (segment (start 123.09 108.35) (end 123.09 100.5) (width 0.25) (layer "B.Cu") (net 39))
 (segment (start 123.13 98.635) (end 123.13 81.291) (width 0.25) (layer "B.Cu") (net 34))
 (segment (start 123.13 81.291) (end 132.937 71.484) (width 0.25) (layer "B.Cu") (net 34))
 (segment (start 123.09 81.331) (end 132.937 71.484) (width 0.25) (layer "B.Cu") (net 34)))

